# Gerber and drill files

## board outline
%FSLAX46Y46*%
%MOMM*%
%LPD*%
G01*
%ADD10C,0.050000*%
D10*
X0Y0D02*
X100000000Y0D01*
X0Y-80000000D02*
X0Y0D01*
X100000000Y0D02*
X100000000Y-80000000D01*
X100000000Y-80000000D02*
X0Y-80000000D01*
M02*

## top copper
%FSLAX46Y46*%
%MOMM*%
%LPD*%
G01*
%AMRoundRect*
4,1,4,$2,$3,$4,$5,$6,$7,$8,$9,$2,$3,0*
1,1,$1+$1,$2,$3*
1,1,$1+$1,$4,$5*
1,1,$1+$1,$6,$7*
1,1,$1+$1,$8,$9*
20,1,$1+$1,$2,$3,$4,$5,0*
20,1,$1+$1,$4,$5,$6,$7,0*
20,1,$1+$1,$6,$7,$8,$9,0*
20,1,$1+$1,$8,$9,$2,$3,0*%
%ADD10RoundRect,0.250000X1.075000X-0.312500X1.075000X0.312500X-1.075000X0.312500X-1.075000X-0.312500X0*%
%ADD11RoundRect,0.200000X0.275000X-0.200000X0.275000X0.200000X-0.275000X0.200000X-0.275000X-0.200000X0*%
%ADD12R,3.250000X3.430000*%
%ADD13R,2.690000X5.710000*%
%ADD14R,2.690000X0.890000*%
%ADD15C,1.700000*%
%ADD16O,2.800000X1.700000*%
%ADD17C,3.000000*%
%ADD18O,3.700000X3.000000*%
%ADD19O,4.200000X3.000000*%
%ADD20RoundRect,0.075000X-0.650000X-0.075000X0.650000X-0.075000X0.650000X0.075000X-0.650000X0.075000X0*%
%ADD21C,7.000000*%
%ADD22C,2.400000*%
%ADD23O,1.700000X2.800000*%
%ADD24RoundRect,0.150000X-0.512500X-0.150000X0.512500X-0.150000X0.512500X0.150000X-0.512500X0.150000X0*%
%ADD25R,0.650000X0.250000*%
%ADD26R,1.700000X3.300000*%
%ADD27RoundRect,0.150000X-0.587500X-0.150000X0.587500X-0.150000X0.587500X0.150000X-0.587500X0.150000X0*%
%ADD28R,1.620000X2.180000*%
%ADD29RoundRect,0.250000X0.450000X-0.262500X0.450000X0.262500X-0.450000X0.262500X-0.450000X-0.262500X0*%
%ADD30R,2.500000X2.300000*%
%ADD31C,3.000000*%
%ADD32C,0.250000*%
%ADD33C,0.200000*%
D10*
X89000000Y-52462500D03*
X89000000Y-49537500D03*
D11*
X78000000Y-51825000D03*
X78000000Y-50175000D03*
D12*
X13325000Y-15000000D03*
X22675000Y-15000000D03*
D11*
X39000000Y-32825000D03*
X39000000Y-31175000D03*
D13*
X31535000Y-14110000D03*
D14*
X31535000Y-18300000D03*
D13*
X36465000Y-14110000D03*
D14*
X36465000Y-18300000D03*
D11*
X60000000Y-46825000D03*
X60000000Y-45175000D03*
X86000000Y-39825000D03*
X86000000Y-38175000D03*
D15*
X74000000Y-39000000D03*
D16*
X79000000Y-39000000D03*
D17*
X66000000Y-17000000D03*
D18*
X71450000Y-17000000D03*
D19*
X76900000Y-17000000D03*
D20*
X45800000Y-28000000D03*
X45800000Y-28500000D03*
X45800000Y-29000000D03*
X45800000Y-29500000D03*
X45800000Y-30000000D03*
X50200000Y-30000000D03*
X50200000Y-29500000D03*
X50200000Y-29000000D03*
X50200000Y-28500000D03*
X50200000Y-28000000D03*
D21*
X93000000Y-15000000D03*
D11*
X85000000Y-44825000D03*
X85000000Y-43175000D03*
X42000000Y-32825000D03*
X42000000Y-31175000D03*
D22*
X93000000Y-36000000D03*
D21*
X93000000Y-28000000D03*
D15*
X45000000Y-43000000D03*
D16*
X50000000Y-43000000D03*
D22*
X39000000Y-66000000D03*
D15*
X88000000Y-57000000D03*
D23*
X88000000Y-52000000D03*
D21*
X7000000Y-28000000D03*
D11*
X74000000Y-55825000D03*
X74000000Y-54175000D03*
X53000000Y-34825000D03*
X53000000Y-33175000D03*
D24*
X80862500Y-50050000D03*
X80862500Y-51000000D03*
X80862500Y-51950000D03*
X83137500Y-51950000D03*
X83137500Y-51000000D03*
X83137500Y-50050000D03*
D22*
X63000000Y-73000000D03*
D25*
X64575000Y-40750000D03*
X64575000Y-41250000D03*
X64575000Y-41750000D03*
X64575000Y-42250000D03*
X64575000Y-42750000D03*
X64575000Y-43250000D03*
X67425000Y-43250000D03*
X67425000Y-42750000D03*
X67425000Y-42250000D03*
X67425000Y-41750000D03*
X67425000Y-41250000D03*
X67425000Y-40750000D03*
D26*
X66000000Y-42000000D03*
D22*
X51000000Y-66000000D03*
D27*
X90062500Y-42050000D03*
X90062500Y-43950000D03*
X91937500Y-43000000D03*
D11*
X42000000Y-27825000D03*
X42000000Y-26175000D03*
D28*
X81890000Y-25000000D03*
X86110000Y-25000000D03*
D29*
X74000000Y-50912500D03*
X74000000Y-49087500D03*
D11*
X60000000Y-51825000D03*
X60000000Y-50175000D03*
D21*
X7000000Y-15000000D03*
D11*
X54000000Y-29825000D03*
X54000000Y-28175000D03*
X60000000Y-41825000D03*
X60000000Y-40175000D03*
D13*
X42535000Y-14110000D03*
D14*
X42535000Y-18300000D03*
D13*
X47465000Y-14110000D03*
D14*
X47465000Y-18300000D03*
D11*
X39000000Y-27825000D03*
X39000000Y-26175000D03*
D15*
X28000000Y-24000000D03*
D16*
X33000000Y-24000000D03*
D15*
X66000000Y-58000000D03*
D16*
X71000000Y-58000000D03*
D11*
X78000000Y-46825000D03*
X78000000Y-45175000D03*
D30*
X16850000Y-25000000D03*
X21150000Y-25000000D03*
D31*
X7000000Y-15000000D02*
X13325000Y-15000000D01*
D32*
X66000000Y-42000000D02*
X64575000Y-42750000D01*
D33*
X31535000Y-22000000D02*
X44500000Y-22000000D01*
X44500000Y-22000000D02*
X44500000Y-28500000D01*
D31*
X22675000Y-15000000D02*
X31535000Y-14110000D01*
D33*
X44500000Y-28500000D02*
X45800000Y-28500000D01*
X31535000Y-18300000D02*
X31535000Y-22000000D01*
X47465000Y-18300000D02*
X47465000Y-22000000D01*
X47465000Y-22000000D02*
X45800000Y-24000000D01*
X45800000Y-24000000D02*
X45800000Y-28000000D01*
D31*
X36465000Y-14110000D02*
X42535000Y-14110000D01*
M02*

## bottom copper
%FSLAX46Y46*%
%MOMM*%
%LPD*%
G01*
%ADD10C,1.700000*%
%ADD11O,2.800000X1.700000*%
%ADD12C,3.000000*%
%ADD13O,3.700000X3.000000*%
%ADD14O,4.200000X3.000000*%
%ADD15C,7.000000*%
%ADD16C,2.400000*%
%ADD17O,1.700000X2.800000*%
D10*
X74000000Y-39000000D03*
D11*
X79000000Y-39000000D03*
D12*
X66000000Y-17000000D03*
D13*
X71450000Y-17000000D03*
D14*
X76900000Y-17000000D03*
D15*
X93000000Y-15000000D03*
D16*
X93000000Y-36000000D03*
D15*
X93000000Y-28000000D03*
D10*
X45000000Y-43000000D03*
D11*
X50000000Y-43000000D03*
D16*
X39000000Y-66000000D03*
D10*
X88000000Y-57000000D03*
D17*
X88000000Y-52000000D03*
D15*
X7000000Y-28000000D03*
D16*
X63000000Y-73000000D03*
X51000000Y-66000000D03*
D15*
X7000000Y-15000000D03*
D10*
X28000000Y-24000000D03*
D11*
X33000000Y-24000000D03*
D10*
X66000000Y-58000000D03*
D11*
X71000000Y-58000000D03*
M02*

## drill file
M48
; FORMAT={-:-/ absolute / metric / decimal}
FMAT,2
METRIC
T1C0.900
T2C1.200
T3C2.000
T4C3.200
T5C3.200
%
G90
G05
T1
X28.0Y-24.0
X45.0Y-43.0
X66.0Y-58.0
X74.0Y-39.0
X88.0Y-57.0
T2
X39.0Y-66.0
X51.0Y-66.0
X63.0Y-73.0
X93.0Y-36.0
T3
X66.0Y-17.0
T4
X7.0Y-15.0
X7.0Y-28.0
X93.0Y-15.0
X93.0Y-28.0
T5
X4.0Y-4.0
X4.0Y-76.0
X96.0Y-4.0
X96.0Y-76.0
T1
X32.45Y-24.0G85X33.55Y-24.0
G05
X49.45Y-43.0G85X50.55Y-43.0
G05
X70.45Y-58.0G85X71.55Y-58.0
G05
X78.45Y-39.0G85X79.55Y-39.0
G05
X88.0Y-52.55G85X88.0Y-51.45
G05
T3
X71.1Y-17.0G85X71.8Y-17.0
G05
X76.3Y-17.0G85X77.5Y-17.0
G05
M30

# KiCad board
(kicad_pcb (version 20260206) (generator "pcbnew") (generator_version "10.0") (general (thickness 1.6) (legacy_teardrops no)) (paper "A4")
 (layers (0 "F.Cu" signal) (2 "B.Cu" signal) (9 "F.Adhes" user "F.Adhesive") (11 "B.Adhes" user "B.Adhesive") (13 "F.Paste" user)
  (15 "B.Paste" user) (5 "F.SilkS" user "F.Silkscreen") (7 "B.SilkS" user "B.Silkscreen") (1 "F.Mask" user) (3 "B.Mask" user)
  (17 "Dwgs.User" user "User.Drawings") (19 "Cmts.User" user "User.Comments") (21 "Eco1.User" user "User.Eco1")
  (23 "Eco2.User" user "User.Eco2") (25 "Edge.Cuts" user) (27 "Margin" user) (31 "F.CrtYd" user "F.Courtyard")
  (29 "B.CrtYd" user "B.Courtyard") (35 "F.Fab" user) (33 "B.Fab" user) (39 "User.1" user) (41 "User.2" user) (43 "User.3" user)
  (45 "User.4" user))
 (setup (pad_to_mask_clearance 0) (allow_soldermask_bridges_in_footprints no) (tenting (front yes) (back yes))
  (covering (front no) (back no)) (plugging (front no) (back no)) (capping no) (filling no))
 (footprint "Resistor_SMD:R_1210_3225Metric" (layer "F.Cu") (at 89 51 90)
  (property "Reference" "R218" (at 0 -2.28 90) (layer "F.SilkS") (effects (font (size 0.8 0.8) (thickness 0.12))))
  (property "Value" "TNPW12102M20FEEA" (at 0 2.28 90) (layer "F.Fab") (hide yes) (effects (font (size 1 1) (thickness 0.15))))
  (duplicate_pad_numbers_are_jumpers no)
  (pad "1" smd roundrect (at -1.4625 0 90) (size 1.125 2.65) (layers "F.Cu" "F.Mask" "F.Paste") (roundrect_rratio 0.222222)
   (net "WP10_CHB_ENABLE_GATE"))
  (pad "2" smd roundrect (at 1.4625 0 90) (size 1.125 2.65) (layers "F.Cu" "F.Mask" "F.Paste") (roundrect_rratio 0.222222)
   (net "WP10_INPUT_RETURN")))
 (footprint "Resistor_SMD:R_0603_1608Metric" (layer "F.Cu") (at 78 51 90)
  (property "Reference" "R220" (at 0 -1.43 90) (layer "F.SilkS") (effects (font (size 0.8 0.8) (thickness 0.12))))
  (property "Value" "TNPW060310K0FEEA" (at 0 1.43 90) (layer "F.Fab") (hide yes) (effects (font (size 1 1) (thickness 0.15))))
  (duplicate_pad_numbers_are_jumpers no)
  (pad "1" smd roundrect (at -0.825 0 90) (size 0.8 0.95) (layers "F.Cu" "F.Mask" "F.Paste") (roundrect_rratio 0.25)
   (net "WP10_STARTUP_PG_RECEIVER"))
  (pad "2" smd roundrect (at 0.825 0 90) (size 0.8 0.95) (layers "F.Cu" "F.Mask" "F.Paste") (roundrect_rratio 0.25)
   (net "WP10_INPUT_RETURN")))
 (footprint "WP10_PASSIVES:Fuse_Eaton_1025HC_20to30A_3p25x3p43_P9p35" (layer "F.Cu") (at 18 15)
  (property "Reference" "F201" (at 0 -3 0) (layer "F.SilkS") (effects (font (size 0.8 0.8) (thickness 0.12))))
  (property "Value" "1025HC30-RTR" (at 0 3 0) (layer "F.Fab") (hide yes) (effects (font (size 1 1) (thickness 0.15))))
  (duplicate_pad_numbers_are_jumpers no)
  (pad "1" smd rect (at -4.675 0) (size 3.25 3.43) (layers "F.Cu" "F.Mask" "F.Paste") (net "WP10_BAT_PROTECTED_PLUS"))
  (pad "2" smd rect (at 4.675 0) (size 3.25 3.43) (layers "F.Cu" "F.Mask" "F.Paste") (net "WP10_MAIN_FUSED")))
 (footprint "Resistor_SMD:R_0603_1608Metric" (layer "F.Cu") (at 39 32 90)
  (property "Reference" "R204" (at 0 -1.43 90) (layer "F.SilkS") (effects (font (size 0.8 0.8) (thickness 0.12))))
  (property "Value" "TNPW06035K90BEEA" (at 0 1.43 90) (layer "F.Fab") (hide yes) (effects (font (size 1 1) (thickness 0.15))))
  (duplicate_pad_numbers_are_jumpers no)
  (pad "1" smd roundrect (at -0.825 0 90) (size 0.8 0.95) (layers "F.Cu" "F.Mask" "F.Paste") (roundrect_rratio 0.25) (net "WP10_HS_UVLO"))
  (pad "2" smd roundrect (at 0.825 0 90) (size 0.8 0.95) (layers "F.Cu" "F.Mask" "F.Paste") (roundrect_rratio 0.25)
   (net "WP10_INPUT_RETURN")))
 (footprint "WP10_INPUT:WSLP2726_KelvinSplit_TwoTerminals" (layer "F.Cu") (at 34 15)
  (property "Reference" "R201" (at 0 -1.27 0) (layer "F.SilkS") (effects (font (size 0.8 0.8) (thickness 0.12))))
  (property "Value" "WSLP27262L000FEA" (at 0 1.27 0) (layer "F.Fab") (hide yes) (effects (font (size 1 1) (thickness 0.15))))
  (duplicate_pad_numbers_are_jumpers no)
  (pad "1" smd rect (at -2.465 -0.89) (size 2.69 5.71) (layers "F.Cu" "F.Mask" "F.Paste") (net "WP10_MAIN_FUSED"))
  (pad "1" smd rect (at -2.465 3.3) (size 2.69 0.89) (layers "F.Cu" "F.Mask" "F.Paste") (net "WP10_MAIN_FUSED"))
  (pad "2" smd rect (at 2.465 -0.89) (size 2.69 5.71) (layers "F.Cu" "F.Mask" "F.Paste") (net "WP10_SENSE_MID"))
  (pad "2" smd rect (at 2.465 3.3) (size 2.69 0.89) (layers "F.Cu" "F.Mask" "F.Paste") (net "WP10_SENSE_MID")))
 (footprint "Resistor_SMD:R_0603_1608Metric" (layer "F.Cu") (at 60 46 90)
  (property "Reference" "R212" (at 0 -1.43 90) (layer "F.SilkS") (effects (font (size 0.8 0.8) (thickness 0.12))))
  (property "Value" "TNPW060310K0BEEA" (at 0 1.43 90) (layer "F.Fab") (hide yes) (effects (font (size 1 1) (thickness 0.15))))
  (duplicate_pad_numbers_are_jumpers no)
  (pad "1" smd roundrect (at -0.825 0 90) (size 0.8 0.95) (layers "F.Cu" "F.Mask" "F.Paste") (roundrect_rratio 0.25)
   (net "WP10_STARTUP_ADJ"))
  (pad "2" smd roundrect (at 0.825 0 90) (size 0.8 0.95) (layers "F.Cu" "F.Mask" "F.Paste") (roundrect_rratio 0.25)
   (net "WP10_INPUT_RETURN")))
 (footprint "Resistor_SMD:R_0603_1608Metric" (layer "F.Cu") (at 86 39 90)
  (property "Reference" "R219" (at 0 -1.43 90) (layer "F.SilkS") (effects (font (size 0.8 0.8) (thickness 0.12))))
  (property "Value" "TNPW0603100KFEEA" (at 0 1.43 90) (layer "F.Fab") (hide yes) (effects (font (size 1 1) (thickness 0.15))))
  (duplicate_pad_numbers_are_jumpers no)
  (pad "1" smd roundrect (at -0.825 0 90) (size 0.8 0.95) (layers "F.Cu" "F.Mask" "F.Paste") (roundrect_rratio 0.25)
   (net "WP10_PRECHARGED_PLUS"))
  (pad "2" smd roundrect (at 0.825 0 90) (size 0.8 0.95) (layers "F.Cu" "F.Mask" "F.Paste") (roundrect_rratio 0.25) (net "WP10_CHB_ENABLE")))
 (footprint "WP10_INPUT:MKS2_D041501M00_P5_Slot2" (layer "F.Cu") (at 74 39)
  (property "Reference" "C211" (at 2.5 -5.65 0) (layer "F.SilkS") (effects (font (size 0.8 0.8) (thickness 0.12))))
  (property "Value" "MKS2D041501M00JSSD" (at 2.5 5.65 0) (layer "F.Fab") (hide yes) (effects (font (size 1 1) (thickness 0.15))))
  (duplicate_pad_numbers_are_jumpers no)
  (pad "1" thru_hole circle (at 0 0) (size 1.7 1.7) (drill 0.9) (layers "*.Cu" "*.Mask") (remove_unused_layers no)
   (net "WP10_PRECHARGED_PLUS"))
  (pad "2" thru_hole oval (at 5 0) (size 2.8 1.7) (drill oval 2 0.9) (layers "*.Cu" "*.Mask") (remove_unused_layers no)
   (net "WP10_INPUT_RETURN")))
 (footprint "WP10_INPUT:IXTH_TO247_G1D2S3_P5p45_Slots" (layer "F.Cu") (at 66 17)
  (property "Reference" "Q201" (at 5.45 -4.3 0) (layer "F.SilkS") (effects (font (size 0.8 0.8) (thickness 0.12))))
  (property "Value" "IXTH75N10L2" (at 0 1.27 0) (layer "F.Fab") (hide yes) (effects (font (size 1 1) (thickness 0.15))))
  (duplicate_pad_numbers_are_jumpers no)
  (pad "1" thru_hole circle (at 0 0) (size 3 3) (drill 2) (layers "*.Cu" "*.Mask") (remove_unused_layers no) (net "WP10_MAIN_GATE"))
  (pad "2" thru_hole oval (at 5.45 0) (size 3.7 3) (drill oval 2.7 2) (layers "*.Cu" "*.Mask") (remove_unused_layers no)
   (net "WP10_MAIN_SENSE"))
  (pad "3" thru_hole oval (at 10.9 0) (size 4.2 3) (drill oval 3.2 2) (layers "*.Cu" "*.Mask") (remove_unused_layers no)
   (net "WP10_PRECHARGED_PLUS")))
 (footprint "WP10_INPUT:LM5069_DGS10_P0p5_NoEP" (layer "F.Cu") (at 48 29)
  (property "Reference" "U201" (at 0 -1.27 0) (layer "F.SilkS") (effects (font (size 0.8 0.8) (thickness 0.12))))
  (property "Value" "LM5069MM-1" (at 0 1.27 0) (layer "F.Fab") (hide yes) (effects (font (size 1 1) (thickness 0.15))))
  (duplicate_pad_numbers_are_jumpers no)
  (pad "1" smd roundrect (at -2.2 -1) (size 1.45 0.3) (layers "F.Cu" "F.Mask" "F.Paste") (roundrect_rratio 0.25) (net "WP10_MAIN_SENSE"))
  (pad "2" smd roundrect (at -2.2 -0.5) (size 1.45 0.3) (layers "F.Cu" "F.Mask" "F.Paste") (roundrect_rratio 0.25) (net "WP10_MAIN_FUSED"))
  (pad "3" smd roundrect (at -2.2 0) (size 1.45 0.3) (layers "F.Cu" "F.Mask" "F.Paste") (roundrect_rratio 0.25) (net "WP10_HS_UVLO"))
  (pad "4" smd roundrect (at -2.2 0.5) (size 1.45 0.3) (layers "F.Cu" "F.Mask" "F.Paste") (roundrect_rratio 0.25) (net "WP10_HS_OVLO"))
  (pad "5" smd roundrect (at -2.2 1) (size 1.45 0.3) (layers "F.Cu" "F.Mask" "F.Paste") (roundrect_rratio 0.25) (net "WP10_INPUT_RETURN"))
  (pad "6" smd roundrect (at 2.2 1) (size 1.45 0.3) (layers "F.Cu" "F.Mask" "F.Paste") (roundrect_rratio 0.25) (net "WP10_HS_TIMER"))
  (pad "7" smd roundrect (at 2.2 0.5) (size 1.45 0.3) (layers "F.Cu" "F.Mask" "F.Paste") (roundrect_rratio 0.25) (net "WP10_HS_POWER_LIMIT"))
  (pad "8" smd roundrect (at 2.2 0) (size 1.45 0.3) (layers "F.Cu" "F.Mask" "F.Paste") (roundrect_rratio 0.25) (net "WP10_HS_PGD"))
  (pad "9" smd roundrect (at 2.2 -0.5) (size 1.45 0.3) (layers "F.Cu" "F.Mask" "F.Paste") (roundrect_rratio 0.25)
   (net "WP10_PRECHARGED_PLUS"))
  (pad "10" smd roundrect (at 2.2 -1) (size 1.45 0.3) (layers "F.Cu" "F.Mask" "F.Paste") (roundrect_rratio 0.25) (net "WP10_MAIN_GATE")))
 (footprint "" (layer "F.Cu") (at 93 15)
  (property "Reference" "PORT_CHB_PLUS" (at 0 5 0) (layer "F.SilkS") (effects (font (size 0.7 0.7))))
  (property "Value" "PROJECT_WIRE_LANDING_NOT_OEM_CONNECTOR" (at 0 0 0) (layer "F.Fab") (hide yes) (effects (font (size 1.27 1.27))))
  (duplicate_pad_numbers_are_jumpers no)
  (pad "1" thru_hole circle (at 0 0) (size 7 7) (drill 3.2) (layers "*.Cu" "*.Mask") (remove_unused_layers no) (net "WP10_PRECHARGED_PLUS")))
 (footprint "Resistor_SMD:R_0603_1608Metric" (layer "F.Cu") (at 85 44 90)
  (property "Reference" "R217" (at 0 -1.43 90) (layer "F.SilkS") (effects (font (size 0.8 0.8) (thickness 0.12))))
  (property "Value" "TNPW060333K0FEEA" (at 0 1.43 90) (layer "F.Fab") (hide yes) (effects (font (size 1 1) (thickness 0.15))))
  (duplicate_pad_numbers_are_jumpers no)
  (pad "1" smd roundrect (at -0.825 0 90) (size 0.8 0.95) (layers "F.Cu" "F.Mask" "F.Paste") (roundrect_rratio 0.25)
   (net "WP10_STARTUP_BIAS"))
  (pad "2" smd roundrect (at 0.825 0 90) (size 0.8 0.95) (layers "F.Cu" "F.Mask" "F.Paste") (roundrect_rratio 0.25)
   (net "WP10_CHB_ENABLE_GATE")))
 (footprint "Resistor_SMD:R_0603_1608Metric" (layer "F.Cu") (at 42 32 90)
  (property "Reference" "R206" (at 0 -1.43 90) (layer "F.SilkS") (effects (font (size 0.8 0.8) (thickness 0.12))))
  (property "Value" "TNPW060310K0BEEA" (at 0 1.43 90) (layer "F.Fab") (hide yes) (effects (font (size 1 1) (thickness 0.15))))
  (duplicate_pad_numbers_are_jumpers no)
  (pad "1" smd roundrect (at -0.825 0 90) (size 0.8 0.95) (layers "F.Cu" "F.Mask" "F.Paste") (roundrect_rratio 0.25) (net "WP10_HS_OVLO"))
  (pad "2" smd roundrect (at 0.825 0 90) (size 0.8 0.95) (layers "F.Cu" "F.Mask" "F.Paste") (roundrect_rratio 0.25)
   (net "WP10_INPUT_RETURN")))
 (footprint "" (layer "F.Cu") (at 93 36)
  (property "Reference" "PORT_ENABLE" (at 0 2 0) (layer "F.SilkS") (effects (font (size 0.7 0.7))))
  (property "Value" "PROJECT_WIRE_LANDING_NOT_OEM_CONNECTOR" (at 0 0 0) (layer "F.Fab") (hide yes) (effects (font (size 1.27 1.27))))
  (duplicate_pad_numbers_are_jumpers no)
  (pad "1" thru_hole circle (at 0 0) (size 2.4 2.4) (drill 1.2) (layers "*.Cu" "*.Mask") (remove_unused_layers no) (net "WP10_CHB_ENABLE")))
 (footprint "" (layer "F.Cu") (at 93 28)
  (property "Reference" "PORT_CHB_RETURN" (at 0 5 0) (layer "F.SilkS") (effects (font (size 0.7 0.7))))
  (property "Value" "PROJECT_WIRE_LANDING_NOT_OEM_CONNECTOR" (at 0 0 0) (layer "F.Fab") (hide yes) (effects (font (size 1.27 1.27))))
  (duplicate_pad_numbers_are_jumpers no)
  (pad "1" thru_hole circle (at 0 0) (size 7 7) (drill 3.2) (layers "*.Cu" "*.Mask") (remove_unused_layers no) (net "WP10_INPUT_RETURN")))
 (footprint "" (layer "F.Cu") (at 96 76)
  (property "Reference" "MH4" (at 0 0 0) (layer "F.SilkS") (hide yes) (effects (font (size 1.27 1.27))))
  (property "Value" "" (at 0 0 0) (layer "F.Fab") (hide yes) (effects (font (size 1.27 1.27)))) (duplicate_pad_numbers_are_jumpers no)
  (pad "" np_thru_hole circle (at 0 0) (size 3.2 3.2) (drill 3.2) (layers "*.Cu" "*.Mask")))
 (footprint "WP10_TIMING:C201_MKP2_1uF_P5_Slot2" (layer "F.Cu") (at 45 43)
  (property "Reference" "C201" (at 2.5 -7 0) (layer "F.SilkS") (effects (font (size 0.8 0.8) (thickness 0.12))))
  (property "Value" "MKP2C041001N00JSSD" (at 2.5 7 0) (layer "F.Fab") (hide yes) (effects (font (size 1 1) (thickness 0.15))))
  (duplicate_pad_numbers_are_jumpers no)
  (pad "1" thru_hole circle (at 0 0) (size 1.7 1.7) (drill 0.9) (layers "*.Cu" "*.Mask") (remove_unused_layers no) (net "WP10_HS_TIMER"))
  (pad "2" thru_hole oval (at 5 0) (size 2.8 1.7) (drill oval 2 0.9) (layers "*.Cu" "*.Mask") (remove_unused_layers no)
   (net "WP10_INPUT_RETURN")))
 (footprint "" (layer "F.Cu") (at 39 66)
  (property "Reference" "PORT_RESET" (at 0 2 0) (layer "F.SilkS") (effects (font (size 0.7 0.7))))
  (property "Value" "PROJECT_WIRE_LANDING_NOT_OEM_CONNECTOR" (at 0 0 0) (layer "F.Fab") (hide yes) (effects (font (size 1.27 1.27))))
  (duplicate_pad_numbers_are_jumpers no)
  (pad "1" thru_hole circle (at 0 0) (size 2.4 2.4) (drill 1.2) (layers "*.Cu" "*.Mask") (remove_unused_layers no) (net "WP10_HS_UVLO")))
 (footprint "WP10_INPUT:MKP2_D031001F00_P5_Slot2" (layer "F.Cu") (at 88 57 90)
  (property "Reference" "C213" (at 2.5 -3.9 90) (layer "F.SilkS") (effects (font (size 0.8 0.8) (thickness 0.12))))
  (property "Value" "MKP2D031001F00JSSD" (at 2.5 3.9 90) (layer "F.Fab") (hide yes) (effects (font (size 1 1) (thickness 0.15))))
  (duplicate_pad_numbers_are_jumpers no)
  (pad "1" thru_hole circle (at 0 0 90) (size 1.7 1.7) (drill 0.9) (layers "*.Cu" "*.Mask") (remove_unused_layers no)
   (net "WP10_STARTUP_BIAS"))
  (pad "2" thru_hole oval (at 5 0 90) (size 2.8 1.7) (drill oval 2 0.9) (layers "*.Cu" "*.Mask") (remove_unused_layers no)
   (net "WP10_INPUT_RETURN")))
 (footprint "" (layer "F.Cu") (at 7 28)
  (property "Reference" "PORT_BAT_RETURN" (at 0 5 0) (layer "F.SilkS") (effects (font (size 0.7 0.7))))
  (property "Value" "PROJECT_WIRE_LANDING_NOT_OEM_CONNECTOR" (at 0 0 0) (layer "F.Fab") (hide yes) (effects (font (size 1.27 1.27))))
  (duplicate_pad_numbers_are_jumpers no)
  (pad "1" thru_hole circle (at 0 0) (size 7 7) (drill 3.2) (layers "*.Cu" "*.Mask") (remove_unused_layers no) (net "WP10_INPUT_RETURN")))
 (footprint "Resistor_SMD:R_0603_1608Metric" (layer "F.Cu") (at 74 55 90)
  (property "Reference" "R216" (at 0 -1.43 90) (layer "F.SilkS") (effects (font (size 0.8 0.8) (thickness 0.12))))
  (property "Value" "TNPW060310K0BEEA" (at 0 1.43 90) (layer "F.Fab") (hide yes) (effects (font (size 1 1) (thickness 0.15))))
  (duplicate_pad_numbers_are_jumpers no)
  (pad "1" smd roundrect (at -0.825 0 90) (size 0.8 0.95) (layers "F.Cu" "F.Mask" "F.Paste") (roundrect_rratio 0.25)
   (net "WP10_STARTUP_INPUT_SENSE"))
  (pad "2" smd roundrect (at 0.825 0 90) (size 0.8 0.95) (layers "F.Cu" "F.Mask" "F.Paste") (roundrect_rratio 0.25)
   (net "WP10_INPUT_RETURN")))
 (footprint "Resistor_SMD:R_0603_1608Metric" (layer "F.Cu") (at 53 34 90)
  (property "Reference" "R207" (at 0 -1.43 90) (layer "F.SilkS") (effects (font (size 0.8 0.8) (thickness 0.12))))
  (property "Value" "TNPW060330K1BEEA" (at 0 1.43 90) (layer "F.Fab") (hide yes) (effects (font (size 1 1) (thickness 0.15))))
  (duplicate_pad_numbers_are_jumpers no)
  (pad "1" smd roundrect (at -0.825 0 90) (size 0.8 0.95) (layers "F.Cu" "F.Mask" "F.Paste") (roundrect_rratio 0.25)
   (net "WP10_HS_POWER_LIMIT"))
  (pad "2" smd roundrect (at 0.825 0 90) (size 0.8 0.95) (layers "F.Cu" "F.Mask" "F.Paste") (roundrect_rratio 0.25)
   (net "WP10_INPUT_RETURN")))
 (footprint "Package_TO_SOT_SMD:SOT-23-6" (layer "F.Cu") (at 82 51)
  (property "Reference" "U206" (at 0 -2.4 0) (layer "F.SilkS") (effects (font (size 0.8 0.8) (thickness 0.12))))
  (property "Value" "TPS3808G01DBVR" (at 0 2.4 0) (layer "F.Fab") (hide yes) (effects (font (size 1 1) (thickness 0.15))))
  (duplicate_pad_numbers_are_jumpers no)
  (pad "1" smd roundrect (at -1.1375 -0.95) (size 1.325 0.6) (layers "F.Cu" "F.Mask" "F.Paste") (roundrect_rratio 0.25)
   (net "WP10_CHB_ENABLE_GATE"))
  (pad "2" smd roundrect (at -1.1375 0) (size 1.325 0.6) (layers "F.Cu" "F.Mask" "F.Paste") (roundrect_rratio 0.25)
   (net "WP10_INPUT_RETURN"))
  (pad "3" smd roundrect (at -1.1375 0.95) (size 1.325 0.6) (layers "F.Cu" "F.Mask" "F.Paste") (roundrect_rratio 0.25)
   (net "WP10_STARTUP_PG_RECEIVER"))
  (pad "4" smd roundrect (at 1.1375 0.95) (size 1.325 0.6) (layers "F.Cu" "F.Mask" "F.Paste") (roundrect_rratio 0.25))
  (pad "5" smd roundrect (at 1.1375 0) (size 1.325 0.6) (layers "F.Cu" "F.Mask" "F.Paste") (roundrect_rratio 0.25)
   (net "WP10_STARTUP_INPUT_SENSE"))
  (pad "6" smd roundrect (at 1.1375 -0.95) (size 1.325 0.6) (layers "F.Cu" "F.Mask" "F.Paste") (roundrect_rratio 0.25)
   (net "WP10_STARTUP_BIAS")))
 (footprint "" (layer "F.Cu") (at 63 73)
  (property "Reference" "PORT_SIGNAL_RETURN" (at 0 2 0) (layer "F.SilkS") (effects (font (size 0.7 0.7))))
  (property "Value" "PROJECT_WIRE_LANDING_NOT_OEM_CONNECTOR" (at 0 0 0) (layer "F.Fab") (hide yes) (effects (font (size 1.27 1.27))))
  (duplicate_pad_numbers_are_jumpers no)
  (pad "1" thru_hole circle (at 0 0) (size 2.4 2.4) (drill 1.2) (layers "*.Cu" "*.Mask") (remove_unused_layers no) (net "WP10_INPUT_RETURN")))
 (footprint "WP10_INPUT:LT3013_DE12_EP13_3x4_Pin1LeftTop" (layer "F.Cu") (at 66 42)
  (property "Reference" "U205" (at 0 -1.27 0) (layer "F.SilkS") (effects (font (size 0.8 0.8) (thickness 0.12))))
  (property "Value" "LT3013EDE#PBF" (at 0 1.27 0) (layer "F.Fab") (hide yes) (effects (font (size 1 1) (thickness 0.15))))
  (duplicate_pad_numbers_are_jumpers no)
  (pad "1" smd rect (at -1.425 -1.25) (size 0.65 0.25) (layers "F.Cu" "F.Mask" "F.Paste"))
  (pad "2" smd rect (at -1.425 -0.75) (size 0.65 0.25) (layers "F.Cu" "F.Mask" "F.Paste") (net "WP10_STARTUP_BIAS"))
  (pad "3" smd rect (at -1.425 -0.25) (size 0.65 0.25) (layers "F.Cu" "F.Mask" "F.Paste") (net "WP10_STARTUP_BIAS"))
  (pad "4" smd rect (at -1.425 0.25) (size 0.65 0.25) (layers "F.Cu" "F.Mask" "F.Paste") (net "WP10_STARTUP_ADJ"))
  (pad "5" smd rect (at -1.425 0.75) (size 0.65 0.25) (layers "F.Cu" "F.Mask" "F.Paste") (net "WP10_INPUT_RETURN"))
  (pad "6" smd rect (at -1.425 1.25) (size 0.65 0.25) (layers "F.Cu" "F.Mask" "F.Paste"))
  (pad "7" smd rect (at 1.425 1.25) (size 0.65 0.25) (layers "F.Cu" "F.Mask" "F.Paste") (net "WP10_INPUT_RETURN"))
  (pad "8" smd rect (at 1.425 0.75) (size 0.65 0.25) (layers "F.Cu" "F.Mask" "F.Paste") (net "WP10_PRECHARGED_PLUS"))
  (pad "9" smd rect (at 1.425 0.25) (size 0.65 0.25) (layers "F.Cu" "F.Mask" "F.Paste"))
  (pad "10" smd rect (at 1.425 -0.25) (size 0.65 0.25) (layers "F.Cu" "F.Mask" "F.Paste") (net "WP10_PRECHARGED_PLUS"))
  (pad "11" smd rect (at 1.425 -0.75) (size 0.65 0.25) (layers "F.Cu" "F.Mask" "F.Paste") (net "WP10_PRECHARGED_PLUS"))
  (pad "12" smd rect (at 1.425 -1.25) (size 0.65 0.25) (layers "F.Cu" "F.Mask" "F.Paste"))
  (pad "13" smd rect (at 0 0) (size 1.7 3.3) (layers "F.Cu" "F.Mask" "F.Paste") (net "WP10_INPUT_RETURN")))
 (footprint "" (layer "F.Cu") (at 4 76)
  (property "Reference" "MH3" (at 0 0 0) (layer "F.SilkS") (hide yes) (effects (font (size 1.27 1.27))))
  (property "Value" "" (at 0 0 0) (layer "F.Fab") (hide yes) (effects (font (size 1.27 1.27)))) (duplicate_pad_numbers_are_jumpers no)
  (pad "" np_thru_hole circle (at 0 0) (size 3.2 3.2) (drill 3.2) (layers "*.Cu" "*.Mask")))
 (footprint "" (layer "F.Cu") (at 96 4)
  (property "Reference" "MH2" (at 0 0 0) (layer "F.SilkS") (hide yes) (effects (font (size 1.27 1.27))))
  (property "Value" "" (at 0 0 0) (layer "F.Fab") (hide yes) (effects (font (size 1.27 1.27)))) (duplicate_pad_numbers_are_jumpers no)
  (pad "" np_thru_hole circle (at 0 0) (size 3.2 3.2) (drill 3.2) (layers "*.Cu" "*.Mask")))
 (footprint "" (layer "F.Cu") (at 51 66)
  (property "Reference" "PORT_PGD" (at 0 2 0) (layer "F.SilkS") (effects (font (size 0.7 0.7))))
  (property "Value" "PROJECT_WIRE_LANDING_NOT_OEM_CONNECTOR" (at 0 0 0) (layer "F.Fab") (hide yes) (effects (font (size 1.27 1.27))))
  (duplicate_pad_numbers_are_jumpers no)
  (pad "1" thru_hole circle (at 0 0) (size 2.4 2.4) (drill 1.2) (layers "*.Cu" "*.Mask") (remove_unused_layers no) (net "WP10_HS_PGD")))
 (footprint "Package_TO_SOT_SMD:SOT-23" (layer "F.Cu") (at 91 43)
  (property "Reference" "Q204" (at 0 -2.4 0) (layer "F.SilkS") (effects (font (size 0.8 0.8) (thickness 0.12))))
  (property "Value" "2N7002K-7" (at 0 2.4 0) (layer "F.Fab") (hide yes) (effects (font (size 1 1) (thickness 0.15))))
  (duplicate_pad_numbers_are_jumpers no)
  (pad "1" smd roundrect (at -0.9375 -0.95) (size 1.475 0.6) (layers "F.Cu" "F.Mask" "F.Paste") (roundrect_rratio 0.25)
   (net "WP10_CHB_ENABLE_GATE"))
  (pad "2" smd roundrect (at -0.9375 0.95) (size 1.475 0.6) (layers "F.Cu" "F.Mask" "F.Paste") (roundrect_rratio 0.25)
   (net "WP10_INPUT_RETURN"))
  (pad "3" smd roundrect (at 0.9375 0) (size 1.475 0.6) (layers "F.Cu" "F.Mask" "F.Paste") (roundrect_rratio 0.25) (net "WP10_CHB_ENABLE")))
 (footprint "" (layer "F.Cu") (at 4 4)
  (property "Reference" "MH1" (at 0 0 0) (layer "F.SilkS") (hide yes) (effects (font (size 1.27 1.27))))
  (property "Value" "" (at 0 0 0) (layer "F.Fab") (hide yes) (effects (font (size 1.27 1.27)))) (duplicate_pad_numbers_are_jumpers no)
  (pad "" np_thru_hole circle (at 0 0) (size 3.2 3.2) (drill 3.2) (layers "*.Cu" "*.Mask")))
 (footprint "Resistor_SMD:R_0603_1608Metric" (layer "F.Cu") (at 42 27 90)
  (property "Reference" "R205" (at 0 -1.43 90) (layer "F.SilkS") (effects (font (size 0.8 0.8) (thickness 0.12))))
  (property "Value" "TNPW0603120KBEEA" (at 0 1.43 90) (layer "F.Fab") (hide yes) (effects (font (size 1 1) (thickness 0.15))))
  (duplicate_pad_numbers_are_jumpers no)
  (pad "1" smd roundrect (at -0.825 0 90) (size 0.8 0.95) (layers "F.Cu" "F.Mask" "F.Paste") (roundrect_rratio 0.25) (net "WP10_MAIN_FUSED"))
  (pad "2" smd roundrect (at 0.825 0 90) (size 0.8 0.95) (layers "F.Cu" "F.Mask" "F.Paste") (roundrect_rratio 0.25) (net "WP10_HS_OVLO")))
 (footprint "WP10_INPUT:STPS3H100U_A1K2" (layer "F.Cu") (at 84 25)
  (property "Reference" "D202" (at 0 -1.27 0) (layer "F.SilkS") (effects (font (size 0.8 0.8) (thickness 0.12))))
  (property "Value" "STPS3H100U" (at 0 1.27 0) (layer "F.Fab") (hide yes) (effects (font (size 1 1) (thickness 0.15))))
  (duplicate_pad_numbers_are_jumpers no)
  (pad "1" smd rect (at -2.11 0) (size 1.62 2.18) (layers "F.Cu" "F.Mask" "F.Paste") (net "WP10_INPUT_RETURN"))
  (pad "2" smd rect (at 2.11 0) (size 1.62 2.18) (layers "F.Cu" "F.Mask" "F.Paste") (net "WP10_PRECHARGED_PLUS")))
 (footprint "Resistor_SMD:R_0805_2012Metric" (layer "F.Cu") (at 74 50 90)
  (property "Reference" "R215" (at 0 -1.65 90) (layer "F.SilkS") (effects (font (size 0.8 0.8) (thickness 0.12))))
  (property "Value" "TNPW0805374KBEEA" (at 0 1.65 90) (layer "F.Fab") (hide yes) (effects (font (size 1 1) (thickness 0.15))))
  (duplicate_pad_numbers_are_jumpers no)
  (pad "1" smd roundrect (at -0.9125 0 90) (size 1.025 1.4) (layers "F.Cu" "F.Mask" "F.Paste") (roundrect_rratio 0.243902)
   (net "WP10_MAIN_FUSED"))
  (pad "2" smd roundrect (at 0.9125 0 90) (size 1.025 1.4) (layers "F.Cu" "F.Mask" "F.Paste") (roundrect_rratio 0.243902)
   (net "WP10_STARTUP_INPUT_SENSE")))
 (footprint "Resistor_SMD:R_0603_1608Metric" (layer "F.Cu") (at 60 51 90)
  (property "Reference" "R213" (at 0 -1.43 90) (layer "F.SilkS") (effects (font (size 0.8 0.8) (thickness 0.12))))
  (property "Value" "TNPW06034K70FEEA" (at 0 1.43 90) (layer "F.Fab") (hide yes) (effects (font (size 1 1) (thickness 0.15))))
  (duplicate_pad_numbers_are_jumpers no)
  (pad "1" smd roundrect (at -0.825 0 90) (size 0.8 0.95) (layers "F.Cu" "F.Mask" "F.Paste") (roundrect_rratio 0.25)
   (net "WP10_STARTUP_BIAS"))
  (pad "2" smd roundrect (at 0.825 0 90) (size 0.8 0.95) (layers "F.Cu" "F.Mask" "F.Paste") (roundrect_rratio 0.25)
   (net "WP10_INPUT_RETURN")))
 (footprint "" (layer "F.Cu") (at 7 15)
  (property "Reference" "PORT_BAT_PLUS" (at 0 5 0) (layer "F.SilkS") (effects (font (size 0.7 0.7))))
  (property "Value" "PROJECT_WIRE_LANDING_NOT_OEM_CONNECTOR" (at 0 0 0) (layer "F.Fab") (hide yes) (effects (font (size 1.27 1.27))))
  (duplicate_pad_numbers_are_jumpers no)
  (pad "1" thru_hole circle (at 0 0) (size 7 7) (drill 3.2) (layers "*.Cu" "*.Mask") (remove_unused_layers no)
   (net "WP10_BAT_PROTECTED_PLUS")))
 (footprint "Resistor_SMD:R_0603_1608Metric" (layer "F.Cu") (at 54 29 90)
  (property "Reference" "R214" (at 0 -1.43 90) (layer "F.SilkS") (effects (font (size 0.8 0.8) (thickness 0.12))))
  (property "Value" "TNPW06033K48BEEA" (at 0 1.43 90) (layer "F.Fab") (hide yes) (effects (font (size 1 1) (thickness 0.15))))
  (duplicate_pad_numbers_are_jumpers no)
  (pad "1" smd roundrect (at -0.825 0 90) (size 0.8 0.95) (layers "F.Cu" "F.Mask" "F.Paste") (roundrect_rratio 0.25)
   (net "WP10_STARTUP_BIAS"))
  (pad "2" smd roundrect (at 0.825 0 90) (size 0.8 0.95) (layers "F.Cu" "F.Mask" "F.Paste") (roundrect_rratio 0.25) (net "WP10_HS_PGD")))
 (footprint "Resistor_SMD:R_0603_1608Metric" (layer "F.Cu") (at 60 41 90)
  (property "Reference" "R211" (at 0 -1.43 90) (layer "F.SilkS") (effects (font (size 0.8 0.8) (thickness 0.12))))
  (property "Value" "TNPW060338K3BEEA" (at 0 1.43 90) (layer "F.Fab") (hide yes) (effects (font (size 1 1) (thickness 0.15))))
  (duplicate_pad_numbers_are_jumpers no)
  (pad "1" smd roundrect (at -0.825 0 90) (size 0.8 0.95) (layers "F.Cu" "F.Mask" "F.Paste") (roundrect_rratio 0.25)
   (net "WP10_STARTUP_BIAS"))
  (pad "2" smd roundrect (at 0.825 0 90) (size 0.8 0.95) (layers "F.Cu" "F.Mask" "F.Paste") (roundrect_rratio 0.25) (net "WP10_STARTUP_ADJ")))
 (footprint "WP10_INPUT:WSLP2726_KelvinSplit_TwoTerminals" (layer "F.Cu") (at 45 15)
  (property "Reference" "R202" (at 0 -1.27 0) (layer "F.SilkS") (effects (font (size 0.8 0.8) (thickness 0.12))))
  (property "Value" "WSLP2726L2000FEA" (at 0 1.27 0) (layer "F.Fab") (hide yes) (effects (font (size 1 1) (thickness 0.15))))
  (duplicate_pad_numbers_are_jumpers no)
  (pad "1" smd rect (at -2.465 -0.89) (size 2.69 5.71) (layers "F.Cu" "F.Mask" "F.Paste") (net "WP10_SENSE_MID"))
  (pad "1" smd rect (at -2.465 3.3) (size 2.69 0.89) (layers "F.Cu" "F.Mask" "F.Paste") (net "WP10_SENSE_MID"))
  (pad "2" smd rect (at 2.465 -0.89) (size 2.69 5.71) (layers "F.Cu" "F.Mask" "F.Paste") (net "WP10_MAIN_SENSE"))
  (pad "2" smd rect (at 2.465 3.3) (size 2.69 0.89) (layers "F.Cu" "F.Mask" "F.Paste") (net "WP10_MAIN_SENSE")))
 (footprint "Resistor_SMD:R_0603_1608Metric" (layer "F.Cu") (at 39 27 90)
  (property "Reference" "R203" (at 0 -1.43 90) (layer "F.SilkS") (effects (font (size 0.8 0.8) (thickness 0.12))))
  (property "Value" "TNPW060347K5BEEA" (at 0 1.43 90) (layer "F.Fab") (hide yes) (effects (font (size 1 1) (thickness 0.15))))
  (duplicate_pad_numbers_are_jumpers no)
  (pad "1" smd roundrect (at -0.825 0 90) (size 0.8 0.95) (layers "F.Cu" "F.Mask" "F.Paste") (roundrect_rratio 0.25) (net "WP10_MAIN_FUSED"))
  (pad "2" smd roundrect (at 0.825 0 90) (size 0.8 0.95) (layers "F.Cu" "F.Mask" "F.Paste") (roundrect_rratio 0.25) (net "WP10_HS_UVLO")))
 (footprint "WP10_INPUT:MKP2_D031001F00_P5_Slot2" (layer "F.Cu") (at 28 24)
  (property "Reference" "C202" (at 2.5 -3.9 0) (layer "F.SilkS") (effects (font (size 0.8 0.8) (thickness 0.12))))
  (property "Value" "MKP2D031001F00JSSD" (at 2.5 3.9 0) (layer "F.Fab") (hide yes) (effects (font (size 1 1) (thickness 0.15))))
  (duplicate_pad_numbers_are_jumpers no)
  (pad "1" thru_hole circle (at 0 0) (size 1.7 1.7) (drill 0.9) (layers "*.Cu" "*.Mask") (remove_unused_layers no) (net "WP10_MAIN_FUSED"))
  (pad "2" thru_hole oval (at 5 0) (size 2.8 1.7) (drill oval 2 0.9) (layers "*.Cu" "*.Mask") (remove_unused_layers no)
   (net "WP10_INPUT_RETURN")))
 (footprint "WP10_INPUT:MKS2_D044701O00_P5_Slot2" (layer "F.Cu") (at 66 58)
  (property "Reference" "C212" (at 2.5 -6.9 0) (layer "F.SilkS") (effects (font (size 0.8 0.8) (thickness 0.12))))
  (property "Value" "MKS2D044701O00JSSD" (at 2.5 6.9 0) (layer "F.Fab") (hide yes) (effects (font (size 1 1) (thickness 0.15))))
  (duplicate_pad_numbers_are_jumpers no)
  (pad "1" thru_hole circle (at 0 0) (size 1.7 1.7) (drill 0.9) (layers "*.Cu" "*.Mask") (remove_unused_layers no) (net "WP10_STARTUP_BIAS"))
  (pad "2" thru_hole oval (at 5 0) (size 2.8 1.7) (drill oval 2 0.9) (layers "*.Cu" "*.Mask") (remove_unused_layers no)
   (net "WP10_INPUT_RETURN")))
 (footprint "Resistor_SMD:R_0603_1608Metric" (layer "F.Cu") (at 78 46 90)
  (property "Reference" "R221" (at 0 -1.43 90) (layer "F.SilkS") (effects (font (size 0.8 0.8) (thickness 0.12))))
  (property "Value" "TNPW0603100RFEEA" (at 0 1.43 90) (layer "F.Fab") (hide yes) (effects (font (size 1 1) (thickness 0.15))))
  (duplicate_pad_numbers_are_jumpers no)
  (pad "1" smd roundrect (at -0.825 0 90) (size 0.8 0.95) (layers "F.Cu" "F.Mask" "F.Paste") (roundrect_rratio 0.25) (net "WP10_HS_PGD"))
  (pad "2" smd roundrect (at 0.825 0 90) (size 0.8 0.95) (layers "F.Cu" "F.Mask" "F.Paste") (roundrect_rratio 0.25)
   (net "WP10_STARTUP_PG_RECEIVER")))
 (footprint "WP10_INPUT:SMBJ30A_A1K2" (layer "F.Cu") (at 19 25)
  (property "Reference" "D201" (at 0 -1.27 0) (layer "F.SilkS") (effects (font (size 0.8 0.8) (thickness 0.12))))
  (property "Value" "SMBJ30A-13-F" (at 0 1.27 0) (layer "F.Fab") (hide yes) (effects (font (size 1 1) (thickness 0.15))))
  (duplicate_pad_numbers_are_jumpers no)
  (pad "1" smd rect (at -2.15 0) (size 2.5 2.3) (layers "F.Cu" "F.Mask" "F.Paste") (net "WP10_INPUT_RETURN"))
  (pad "2" smd rect (at 2.15 0) (size 2.5 2.3) (layers "F.Cu" "F.Mask" "F.Paste") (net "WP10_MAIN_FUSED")))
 (gr_line (start 0 0) (end 100 0) (stroke (width 0.05) (type default)) (layer "Edge.Cuts"))
 (gr_line (start 0 80) (end 0 0) (stroke (width 0.05) (type default)) (layer "Edge.Cuts"))
 (gr_line (start 100 0) (end 100 80) (stroke (width 0.05) (type default)) (layer "Edge.Cuts"))
 (gr_line (start 100 80) (end 0 80) (stroke (width 0.05) (type default)) (layer "Edge.Cuts"))
 (segment (start 7 15) (end 13.325 15) (width 3) (layer "F.Cu") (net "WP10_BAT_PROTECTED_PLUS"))
 (segment (start 66 42) (end 64.575 42.75) (width 0.25) (layer "F.Cu") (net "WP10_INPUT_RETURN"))
 (segment (start 31.535 22) (end 44.5 22) (width 0.2) (layer "F.Cu") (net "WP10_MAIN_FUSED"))
 (segment (start 44.5 22) (end 44.5 28.5) (width 0.2) (layer "F.Cu") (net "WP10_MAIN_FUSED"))
 (segment (start 22.675 15) (end 31.535 14.11) (width 3) (layer "F.Cu") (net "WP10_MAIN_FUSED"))
 (segment (start 44.5 28.5) (end 45.8 28.5) (width 0.2) (layer "F.Cu") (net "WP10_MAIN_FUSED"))
 (segment (start 31.535 18.3) (end 31.535 22) (width 0.2) (layer "F.Cu") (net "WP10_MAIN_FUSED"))
 (segment (start 47.465 18.3) (end 47.465 22) (width 0.2) (layer "F.Cu") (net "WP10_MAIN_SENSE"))
 (segment (start 47.465 22) (end 45.8 24) (width 0.2) (layer "F.Cu") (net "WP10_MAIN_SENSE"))
 (segment (start 45.8 24) (end 45.8 28) (width 0.2) (layer "F.Cu") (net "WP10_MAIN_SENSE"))
 (segment (start 36.465 14.11) (end 42.535 14.11) (width 3) (layer "F.Cu") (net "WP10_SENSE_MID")))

